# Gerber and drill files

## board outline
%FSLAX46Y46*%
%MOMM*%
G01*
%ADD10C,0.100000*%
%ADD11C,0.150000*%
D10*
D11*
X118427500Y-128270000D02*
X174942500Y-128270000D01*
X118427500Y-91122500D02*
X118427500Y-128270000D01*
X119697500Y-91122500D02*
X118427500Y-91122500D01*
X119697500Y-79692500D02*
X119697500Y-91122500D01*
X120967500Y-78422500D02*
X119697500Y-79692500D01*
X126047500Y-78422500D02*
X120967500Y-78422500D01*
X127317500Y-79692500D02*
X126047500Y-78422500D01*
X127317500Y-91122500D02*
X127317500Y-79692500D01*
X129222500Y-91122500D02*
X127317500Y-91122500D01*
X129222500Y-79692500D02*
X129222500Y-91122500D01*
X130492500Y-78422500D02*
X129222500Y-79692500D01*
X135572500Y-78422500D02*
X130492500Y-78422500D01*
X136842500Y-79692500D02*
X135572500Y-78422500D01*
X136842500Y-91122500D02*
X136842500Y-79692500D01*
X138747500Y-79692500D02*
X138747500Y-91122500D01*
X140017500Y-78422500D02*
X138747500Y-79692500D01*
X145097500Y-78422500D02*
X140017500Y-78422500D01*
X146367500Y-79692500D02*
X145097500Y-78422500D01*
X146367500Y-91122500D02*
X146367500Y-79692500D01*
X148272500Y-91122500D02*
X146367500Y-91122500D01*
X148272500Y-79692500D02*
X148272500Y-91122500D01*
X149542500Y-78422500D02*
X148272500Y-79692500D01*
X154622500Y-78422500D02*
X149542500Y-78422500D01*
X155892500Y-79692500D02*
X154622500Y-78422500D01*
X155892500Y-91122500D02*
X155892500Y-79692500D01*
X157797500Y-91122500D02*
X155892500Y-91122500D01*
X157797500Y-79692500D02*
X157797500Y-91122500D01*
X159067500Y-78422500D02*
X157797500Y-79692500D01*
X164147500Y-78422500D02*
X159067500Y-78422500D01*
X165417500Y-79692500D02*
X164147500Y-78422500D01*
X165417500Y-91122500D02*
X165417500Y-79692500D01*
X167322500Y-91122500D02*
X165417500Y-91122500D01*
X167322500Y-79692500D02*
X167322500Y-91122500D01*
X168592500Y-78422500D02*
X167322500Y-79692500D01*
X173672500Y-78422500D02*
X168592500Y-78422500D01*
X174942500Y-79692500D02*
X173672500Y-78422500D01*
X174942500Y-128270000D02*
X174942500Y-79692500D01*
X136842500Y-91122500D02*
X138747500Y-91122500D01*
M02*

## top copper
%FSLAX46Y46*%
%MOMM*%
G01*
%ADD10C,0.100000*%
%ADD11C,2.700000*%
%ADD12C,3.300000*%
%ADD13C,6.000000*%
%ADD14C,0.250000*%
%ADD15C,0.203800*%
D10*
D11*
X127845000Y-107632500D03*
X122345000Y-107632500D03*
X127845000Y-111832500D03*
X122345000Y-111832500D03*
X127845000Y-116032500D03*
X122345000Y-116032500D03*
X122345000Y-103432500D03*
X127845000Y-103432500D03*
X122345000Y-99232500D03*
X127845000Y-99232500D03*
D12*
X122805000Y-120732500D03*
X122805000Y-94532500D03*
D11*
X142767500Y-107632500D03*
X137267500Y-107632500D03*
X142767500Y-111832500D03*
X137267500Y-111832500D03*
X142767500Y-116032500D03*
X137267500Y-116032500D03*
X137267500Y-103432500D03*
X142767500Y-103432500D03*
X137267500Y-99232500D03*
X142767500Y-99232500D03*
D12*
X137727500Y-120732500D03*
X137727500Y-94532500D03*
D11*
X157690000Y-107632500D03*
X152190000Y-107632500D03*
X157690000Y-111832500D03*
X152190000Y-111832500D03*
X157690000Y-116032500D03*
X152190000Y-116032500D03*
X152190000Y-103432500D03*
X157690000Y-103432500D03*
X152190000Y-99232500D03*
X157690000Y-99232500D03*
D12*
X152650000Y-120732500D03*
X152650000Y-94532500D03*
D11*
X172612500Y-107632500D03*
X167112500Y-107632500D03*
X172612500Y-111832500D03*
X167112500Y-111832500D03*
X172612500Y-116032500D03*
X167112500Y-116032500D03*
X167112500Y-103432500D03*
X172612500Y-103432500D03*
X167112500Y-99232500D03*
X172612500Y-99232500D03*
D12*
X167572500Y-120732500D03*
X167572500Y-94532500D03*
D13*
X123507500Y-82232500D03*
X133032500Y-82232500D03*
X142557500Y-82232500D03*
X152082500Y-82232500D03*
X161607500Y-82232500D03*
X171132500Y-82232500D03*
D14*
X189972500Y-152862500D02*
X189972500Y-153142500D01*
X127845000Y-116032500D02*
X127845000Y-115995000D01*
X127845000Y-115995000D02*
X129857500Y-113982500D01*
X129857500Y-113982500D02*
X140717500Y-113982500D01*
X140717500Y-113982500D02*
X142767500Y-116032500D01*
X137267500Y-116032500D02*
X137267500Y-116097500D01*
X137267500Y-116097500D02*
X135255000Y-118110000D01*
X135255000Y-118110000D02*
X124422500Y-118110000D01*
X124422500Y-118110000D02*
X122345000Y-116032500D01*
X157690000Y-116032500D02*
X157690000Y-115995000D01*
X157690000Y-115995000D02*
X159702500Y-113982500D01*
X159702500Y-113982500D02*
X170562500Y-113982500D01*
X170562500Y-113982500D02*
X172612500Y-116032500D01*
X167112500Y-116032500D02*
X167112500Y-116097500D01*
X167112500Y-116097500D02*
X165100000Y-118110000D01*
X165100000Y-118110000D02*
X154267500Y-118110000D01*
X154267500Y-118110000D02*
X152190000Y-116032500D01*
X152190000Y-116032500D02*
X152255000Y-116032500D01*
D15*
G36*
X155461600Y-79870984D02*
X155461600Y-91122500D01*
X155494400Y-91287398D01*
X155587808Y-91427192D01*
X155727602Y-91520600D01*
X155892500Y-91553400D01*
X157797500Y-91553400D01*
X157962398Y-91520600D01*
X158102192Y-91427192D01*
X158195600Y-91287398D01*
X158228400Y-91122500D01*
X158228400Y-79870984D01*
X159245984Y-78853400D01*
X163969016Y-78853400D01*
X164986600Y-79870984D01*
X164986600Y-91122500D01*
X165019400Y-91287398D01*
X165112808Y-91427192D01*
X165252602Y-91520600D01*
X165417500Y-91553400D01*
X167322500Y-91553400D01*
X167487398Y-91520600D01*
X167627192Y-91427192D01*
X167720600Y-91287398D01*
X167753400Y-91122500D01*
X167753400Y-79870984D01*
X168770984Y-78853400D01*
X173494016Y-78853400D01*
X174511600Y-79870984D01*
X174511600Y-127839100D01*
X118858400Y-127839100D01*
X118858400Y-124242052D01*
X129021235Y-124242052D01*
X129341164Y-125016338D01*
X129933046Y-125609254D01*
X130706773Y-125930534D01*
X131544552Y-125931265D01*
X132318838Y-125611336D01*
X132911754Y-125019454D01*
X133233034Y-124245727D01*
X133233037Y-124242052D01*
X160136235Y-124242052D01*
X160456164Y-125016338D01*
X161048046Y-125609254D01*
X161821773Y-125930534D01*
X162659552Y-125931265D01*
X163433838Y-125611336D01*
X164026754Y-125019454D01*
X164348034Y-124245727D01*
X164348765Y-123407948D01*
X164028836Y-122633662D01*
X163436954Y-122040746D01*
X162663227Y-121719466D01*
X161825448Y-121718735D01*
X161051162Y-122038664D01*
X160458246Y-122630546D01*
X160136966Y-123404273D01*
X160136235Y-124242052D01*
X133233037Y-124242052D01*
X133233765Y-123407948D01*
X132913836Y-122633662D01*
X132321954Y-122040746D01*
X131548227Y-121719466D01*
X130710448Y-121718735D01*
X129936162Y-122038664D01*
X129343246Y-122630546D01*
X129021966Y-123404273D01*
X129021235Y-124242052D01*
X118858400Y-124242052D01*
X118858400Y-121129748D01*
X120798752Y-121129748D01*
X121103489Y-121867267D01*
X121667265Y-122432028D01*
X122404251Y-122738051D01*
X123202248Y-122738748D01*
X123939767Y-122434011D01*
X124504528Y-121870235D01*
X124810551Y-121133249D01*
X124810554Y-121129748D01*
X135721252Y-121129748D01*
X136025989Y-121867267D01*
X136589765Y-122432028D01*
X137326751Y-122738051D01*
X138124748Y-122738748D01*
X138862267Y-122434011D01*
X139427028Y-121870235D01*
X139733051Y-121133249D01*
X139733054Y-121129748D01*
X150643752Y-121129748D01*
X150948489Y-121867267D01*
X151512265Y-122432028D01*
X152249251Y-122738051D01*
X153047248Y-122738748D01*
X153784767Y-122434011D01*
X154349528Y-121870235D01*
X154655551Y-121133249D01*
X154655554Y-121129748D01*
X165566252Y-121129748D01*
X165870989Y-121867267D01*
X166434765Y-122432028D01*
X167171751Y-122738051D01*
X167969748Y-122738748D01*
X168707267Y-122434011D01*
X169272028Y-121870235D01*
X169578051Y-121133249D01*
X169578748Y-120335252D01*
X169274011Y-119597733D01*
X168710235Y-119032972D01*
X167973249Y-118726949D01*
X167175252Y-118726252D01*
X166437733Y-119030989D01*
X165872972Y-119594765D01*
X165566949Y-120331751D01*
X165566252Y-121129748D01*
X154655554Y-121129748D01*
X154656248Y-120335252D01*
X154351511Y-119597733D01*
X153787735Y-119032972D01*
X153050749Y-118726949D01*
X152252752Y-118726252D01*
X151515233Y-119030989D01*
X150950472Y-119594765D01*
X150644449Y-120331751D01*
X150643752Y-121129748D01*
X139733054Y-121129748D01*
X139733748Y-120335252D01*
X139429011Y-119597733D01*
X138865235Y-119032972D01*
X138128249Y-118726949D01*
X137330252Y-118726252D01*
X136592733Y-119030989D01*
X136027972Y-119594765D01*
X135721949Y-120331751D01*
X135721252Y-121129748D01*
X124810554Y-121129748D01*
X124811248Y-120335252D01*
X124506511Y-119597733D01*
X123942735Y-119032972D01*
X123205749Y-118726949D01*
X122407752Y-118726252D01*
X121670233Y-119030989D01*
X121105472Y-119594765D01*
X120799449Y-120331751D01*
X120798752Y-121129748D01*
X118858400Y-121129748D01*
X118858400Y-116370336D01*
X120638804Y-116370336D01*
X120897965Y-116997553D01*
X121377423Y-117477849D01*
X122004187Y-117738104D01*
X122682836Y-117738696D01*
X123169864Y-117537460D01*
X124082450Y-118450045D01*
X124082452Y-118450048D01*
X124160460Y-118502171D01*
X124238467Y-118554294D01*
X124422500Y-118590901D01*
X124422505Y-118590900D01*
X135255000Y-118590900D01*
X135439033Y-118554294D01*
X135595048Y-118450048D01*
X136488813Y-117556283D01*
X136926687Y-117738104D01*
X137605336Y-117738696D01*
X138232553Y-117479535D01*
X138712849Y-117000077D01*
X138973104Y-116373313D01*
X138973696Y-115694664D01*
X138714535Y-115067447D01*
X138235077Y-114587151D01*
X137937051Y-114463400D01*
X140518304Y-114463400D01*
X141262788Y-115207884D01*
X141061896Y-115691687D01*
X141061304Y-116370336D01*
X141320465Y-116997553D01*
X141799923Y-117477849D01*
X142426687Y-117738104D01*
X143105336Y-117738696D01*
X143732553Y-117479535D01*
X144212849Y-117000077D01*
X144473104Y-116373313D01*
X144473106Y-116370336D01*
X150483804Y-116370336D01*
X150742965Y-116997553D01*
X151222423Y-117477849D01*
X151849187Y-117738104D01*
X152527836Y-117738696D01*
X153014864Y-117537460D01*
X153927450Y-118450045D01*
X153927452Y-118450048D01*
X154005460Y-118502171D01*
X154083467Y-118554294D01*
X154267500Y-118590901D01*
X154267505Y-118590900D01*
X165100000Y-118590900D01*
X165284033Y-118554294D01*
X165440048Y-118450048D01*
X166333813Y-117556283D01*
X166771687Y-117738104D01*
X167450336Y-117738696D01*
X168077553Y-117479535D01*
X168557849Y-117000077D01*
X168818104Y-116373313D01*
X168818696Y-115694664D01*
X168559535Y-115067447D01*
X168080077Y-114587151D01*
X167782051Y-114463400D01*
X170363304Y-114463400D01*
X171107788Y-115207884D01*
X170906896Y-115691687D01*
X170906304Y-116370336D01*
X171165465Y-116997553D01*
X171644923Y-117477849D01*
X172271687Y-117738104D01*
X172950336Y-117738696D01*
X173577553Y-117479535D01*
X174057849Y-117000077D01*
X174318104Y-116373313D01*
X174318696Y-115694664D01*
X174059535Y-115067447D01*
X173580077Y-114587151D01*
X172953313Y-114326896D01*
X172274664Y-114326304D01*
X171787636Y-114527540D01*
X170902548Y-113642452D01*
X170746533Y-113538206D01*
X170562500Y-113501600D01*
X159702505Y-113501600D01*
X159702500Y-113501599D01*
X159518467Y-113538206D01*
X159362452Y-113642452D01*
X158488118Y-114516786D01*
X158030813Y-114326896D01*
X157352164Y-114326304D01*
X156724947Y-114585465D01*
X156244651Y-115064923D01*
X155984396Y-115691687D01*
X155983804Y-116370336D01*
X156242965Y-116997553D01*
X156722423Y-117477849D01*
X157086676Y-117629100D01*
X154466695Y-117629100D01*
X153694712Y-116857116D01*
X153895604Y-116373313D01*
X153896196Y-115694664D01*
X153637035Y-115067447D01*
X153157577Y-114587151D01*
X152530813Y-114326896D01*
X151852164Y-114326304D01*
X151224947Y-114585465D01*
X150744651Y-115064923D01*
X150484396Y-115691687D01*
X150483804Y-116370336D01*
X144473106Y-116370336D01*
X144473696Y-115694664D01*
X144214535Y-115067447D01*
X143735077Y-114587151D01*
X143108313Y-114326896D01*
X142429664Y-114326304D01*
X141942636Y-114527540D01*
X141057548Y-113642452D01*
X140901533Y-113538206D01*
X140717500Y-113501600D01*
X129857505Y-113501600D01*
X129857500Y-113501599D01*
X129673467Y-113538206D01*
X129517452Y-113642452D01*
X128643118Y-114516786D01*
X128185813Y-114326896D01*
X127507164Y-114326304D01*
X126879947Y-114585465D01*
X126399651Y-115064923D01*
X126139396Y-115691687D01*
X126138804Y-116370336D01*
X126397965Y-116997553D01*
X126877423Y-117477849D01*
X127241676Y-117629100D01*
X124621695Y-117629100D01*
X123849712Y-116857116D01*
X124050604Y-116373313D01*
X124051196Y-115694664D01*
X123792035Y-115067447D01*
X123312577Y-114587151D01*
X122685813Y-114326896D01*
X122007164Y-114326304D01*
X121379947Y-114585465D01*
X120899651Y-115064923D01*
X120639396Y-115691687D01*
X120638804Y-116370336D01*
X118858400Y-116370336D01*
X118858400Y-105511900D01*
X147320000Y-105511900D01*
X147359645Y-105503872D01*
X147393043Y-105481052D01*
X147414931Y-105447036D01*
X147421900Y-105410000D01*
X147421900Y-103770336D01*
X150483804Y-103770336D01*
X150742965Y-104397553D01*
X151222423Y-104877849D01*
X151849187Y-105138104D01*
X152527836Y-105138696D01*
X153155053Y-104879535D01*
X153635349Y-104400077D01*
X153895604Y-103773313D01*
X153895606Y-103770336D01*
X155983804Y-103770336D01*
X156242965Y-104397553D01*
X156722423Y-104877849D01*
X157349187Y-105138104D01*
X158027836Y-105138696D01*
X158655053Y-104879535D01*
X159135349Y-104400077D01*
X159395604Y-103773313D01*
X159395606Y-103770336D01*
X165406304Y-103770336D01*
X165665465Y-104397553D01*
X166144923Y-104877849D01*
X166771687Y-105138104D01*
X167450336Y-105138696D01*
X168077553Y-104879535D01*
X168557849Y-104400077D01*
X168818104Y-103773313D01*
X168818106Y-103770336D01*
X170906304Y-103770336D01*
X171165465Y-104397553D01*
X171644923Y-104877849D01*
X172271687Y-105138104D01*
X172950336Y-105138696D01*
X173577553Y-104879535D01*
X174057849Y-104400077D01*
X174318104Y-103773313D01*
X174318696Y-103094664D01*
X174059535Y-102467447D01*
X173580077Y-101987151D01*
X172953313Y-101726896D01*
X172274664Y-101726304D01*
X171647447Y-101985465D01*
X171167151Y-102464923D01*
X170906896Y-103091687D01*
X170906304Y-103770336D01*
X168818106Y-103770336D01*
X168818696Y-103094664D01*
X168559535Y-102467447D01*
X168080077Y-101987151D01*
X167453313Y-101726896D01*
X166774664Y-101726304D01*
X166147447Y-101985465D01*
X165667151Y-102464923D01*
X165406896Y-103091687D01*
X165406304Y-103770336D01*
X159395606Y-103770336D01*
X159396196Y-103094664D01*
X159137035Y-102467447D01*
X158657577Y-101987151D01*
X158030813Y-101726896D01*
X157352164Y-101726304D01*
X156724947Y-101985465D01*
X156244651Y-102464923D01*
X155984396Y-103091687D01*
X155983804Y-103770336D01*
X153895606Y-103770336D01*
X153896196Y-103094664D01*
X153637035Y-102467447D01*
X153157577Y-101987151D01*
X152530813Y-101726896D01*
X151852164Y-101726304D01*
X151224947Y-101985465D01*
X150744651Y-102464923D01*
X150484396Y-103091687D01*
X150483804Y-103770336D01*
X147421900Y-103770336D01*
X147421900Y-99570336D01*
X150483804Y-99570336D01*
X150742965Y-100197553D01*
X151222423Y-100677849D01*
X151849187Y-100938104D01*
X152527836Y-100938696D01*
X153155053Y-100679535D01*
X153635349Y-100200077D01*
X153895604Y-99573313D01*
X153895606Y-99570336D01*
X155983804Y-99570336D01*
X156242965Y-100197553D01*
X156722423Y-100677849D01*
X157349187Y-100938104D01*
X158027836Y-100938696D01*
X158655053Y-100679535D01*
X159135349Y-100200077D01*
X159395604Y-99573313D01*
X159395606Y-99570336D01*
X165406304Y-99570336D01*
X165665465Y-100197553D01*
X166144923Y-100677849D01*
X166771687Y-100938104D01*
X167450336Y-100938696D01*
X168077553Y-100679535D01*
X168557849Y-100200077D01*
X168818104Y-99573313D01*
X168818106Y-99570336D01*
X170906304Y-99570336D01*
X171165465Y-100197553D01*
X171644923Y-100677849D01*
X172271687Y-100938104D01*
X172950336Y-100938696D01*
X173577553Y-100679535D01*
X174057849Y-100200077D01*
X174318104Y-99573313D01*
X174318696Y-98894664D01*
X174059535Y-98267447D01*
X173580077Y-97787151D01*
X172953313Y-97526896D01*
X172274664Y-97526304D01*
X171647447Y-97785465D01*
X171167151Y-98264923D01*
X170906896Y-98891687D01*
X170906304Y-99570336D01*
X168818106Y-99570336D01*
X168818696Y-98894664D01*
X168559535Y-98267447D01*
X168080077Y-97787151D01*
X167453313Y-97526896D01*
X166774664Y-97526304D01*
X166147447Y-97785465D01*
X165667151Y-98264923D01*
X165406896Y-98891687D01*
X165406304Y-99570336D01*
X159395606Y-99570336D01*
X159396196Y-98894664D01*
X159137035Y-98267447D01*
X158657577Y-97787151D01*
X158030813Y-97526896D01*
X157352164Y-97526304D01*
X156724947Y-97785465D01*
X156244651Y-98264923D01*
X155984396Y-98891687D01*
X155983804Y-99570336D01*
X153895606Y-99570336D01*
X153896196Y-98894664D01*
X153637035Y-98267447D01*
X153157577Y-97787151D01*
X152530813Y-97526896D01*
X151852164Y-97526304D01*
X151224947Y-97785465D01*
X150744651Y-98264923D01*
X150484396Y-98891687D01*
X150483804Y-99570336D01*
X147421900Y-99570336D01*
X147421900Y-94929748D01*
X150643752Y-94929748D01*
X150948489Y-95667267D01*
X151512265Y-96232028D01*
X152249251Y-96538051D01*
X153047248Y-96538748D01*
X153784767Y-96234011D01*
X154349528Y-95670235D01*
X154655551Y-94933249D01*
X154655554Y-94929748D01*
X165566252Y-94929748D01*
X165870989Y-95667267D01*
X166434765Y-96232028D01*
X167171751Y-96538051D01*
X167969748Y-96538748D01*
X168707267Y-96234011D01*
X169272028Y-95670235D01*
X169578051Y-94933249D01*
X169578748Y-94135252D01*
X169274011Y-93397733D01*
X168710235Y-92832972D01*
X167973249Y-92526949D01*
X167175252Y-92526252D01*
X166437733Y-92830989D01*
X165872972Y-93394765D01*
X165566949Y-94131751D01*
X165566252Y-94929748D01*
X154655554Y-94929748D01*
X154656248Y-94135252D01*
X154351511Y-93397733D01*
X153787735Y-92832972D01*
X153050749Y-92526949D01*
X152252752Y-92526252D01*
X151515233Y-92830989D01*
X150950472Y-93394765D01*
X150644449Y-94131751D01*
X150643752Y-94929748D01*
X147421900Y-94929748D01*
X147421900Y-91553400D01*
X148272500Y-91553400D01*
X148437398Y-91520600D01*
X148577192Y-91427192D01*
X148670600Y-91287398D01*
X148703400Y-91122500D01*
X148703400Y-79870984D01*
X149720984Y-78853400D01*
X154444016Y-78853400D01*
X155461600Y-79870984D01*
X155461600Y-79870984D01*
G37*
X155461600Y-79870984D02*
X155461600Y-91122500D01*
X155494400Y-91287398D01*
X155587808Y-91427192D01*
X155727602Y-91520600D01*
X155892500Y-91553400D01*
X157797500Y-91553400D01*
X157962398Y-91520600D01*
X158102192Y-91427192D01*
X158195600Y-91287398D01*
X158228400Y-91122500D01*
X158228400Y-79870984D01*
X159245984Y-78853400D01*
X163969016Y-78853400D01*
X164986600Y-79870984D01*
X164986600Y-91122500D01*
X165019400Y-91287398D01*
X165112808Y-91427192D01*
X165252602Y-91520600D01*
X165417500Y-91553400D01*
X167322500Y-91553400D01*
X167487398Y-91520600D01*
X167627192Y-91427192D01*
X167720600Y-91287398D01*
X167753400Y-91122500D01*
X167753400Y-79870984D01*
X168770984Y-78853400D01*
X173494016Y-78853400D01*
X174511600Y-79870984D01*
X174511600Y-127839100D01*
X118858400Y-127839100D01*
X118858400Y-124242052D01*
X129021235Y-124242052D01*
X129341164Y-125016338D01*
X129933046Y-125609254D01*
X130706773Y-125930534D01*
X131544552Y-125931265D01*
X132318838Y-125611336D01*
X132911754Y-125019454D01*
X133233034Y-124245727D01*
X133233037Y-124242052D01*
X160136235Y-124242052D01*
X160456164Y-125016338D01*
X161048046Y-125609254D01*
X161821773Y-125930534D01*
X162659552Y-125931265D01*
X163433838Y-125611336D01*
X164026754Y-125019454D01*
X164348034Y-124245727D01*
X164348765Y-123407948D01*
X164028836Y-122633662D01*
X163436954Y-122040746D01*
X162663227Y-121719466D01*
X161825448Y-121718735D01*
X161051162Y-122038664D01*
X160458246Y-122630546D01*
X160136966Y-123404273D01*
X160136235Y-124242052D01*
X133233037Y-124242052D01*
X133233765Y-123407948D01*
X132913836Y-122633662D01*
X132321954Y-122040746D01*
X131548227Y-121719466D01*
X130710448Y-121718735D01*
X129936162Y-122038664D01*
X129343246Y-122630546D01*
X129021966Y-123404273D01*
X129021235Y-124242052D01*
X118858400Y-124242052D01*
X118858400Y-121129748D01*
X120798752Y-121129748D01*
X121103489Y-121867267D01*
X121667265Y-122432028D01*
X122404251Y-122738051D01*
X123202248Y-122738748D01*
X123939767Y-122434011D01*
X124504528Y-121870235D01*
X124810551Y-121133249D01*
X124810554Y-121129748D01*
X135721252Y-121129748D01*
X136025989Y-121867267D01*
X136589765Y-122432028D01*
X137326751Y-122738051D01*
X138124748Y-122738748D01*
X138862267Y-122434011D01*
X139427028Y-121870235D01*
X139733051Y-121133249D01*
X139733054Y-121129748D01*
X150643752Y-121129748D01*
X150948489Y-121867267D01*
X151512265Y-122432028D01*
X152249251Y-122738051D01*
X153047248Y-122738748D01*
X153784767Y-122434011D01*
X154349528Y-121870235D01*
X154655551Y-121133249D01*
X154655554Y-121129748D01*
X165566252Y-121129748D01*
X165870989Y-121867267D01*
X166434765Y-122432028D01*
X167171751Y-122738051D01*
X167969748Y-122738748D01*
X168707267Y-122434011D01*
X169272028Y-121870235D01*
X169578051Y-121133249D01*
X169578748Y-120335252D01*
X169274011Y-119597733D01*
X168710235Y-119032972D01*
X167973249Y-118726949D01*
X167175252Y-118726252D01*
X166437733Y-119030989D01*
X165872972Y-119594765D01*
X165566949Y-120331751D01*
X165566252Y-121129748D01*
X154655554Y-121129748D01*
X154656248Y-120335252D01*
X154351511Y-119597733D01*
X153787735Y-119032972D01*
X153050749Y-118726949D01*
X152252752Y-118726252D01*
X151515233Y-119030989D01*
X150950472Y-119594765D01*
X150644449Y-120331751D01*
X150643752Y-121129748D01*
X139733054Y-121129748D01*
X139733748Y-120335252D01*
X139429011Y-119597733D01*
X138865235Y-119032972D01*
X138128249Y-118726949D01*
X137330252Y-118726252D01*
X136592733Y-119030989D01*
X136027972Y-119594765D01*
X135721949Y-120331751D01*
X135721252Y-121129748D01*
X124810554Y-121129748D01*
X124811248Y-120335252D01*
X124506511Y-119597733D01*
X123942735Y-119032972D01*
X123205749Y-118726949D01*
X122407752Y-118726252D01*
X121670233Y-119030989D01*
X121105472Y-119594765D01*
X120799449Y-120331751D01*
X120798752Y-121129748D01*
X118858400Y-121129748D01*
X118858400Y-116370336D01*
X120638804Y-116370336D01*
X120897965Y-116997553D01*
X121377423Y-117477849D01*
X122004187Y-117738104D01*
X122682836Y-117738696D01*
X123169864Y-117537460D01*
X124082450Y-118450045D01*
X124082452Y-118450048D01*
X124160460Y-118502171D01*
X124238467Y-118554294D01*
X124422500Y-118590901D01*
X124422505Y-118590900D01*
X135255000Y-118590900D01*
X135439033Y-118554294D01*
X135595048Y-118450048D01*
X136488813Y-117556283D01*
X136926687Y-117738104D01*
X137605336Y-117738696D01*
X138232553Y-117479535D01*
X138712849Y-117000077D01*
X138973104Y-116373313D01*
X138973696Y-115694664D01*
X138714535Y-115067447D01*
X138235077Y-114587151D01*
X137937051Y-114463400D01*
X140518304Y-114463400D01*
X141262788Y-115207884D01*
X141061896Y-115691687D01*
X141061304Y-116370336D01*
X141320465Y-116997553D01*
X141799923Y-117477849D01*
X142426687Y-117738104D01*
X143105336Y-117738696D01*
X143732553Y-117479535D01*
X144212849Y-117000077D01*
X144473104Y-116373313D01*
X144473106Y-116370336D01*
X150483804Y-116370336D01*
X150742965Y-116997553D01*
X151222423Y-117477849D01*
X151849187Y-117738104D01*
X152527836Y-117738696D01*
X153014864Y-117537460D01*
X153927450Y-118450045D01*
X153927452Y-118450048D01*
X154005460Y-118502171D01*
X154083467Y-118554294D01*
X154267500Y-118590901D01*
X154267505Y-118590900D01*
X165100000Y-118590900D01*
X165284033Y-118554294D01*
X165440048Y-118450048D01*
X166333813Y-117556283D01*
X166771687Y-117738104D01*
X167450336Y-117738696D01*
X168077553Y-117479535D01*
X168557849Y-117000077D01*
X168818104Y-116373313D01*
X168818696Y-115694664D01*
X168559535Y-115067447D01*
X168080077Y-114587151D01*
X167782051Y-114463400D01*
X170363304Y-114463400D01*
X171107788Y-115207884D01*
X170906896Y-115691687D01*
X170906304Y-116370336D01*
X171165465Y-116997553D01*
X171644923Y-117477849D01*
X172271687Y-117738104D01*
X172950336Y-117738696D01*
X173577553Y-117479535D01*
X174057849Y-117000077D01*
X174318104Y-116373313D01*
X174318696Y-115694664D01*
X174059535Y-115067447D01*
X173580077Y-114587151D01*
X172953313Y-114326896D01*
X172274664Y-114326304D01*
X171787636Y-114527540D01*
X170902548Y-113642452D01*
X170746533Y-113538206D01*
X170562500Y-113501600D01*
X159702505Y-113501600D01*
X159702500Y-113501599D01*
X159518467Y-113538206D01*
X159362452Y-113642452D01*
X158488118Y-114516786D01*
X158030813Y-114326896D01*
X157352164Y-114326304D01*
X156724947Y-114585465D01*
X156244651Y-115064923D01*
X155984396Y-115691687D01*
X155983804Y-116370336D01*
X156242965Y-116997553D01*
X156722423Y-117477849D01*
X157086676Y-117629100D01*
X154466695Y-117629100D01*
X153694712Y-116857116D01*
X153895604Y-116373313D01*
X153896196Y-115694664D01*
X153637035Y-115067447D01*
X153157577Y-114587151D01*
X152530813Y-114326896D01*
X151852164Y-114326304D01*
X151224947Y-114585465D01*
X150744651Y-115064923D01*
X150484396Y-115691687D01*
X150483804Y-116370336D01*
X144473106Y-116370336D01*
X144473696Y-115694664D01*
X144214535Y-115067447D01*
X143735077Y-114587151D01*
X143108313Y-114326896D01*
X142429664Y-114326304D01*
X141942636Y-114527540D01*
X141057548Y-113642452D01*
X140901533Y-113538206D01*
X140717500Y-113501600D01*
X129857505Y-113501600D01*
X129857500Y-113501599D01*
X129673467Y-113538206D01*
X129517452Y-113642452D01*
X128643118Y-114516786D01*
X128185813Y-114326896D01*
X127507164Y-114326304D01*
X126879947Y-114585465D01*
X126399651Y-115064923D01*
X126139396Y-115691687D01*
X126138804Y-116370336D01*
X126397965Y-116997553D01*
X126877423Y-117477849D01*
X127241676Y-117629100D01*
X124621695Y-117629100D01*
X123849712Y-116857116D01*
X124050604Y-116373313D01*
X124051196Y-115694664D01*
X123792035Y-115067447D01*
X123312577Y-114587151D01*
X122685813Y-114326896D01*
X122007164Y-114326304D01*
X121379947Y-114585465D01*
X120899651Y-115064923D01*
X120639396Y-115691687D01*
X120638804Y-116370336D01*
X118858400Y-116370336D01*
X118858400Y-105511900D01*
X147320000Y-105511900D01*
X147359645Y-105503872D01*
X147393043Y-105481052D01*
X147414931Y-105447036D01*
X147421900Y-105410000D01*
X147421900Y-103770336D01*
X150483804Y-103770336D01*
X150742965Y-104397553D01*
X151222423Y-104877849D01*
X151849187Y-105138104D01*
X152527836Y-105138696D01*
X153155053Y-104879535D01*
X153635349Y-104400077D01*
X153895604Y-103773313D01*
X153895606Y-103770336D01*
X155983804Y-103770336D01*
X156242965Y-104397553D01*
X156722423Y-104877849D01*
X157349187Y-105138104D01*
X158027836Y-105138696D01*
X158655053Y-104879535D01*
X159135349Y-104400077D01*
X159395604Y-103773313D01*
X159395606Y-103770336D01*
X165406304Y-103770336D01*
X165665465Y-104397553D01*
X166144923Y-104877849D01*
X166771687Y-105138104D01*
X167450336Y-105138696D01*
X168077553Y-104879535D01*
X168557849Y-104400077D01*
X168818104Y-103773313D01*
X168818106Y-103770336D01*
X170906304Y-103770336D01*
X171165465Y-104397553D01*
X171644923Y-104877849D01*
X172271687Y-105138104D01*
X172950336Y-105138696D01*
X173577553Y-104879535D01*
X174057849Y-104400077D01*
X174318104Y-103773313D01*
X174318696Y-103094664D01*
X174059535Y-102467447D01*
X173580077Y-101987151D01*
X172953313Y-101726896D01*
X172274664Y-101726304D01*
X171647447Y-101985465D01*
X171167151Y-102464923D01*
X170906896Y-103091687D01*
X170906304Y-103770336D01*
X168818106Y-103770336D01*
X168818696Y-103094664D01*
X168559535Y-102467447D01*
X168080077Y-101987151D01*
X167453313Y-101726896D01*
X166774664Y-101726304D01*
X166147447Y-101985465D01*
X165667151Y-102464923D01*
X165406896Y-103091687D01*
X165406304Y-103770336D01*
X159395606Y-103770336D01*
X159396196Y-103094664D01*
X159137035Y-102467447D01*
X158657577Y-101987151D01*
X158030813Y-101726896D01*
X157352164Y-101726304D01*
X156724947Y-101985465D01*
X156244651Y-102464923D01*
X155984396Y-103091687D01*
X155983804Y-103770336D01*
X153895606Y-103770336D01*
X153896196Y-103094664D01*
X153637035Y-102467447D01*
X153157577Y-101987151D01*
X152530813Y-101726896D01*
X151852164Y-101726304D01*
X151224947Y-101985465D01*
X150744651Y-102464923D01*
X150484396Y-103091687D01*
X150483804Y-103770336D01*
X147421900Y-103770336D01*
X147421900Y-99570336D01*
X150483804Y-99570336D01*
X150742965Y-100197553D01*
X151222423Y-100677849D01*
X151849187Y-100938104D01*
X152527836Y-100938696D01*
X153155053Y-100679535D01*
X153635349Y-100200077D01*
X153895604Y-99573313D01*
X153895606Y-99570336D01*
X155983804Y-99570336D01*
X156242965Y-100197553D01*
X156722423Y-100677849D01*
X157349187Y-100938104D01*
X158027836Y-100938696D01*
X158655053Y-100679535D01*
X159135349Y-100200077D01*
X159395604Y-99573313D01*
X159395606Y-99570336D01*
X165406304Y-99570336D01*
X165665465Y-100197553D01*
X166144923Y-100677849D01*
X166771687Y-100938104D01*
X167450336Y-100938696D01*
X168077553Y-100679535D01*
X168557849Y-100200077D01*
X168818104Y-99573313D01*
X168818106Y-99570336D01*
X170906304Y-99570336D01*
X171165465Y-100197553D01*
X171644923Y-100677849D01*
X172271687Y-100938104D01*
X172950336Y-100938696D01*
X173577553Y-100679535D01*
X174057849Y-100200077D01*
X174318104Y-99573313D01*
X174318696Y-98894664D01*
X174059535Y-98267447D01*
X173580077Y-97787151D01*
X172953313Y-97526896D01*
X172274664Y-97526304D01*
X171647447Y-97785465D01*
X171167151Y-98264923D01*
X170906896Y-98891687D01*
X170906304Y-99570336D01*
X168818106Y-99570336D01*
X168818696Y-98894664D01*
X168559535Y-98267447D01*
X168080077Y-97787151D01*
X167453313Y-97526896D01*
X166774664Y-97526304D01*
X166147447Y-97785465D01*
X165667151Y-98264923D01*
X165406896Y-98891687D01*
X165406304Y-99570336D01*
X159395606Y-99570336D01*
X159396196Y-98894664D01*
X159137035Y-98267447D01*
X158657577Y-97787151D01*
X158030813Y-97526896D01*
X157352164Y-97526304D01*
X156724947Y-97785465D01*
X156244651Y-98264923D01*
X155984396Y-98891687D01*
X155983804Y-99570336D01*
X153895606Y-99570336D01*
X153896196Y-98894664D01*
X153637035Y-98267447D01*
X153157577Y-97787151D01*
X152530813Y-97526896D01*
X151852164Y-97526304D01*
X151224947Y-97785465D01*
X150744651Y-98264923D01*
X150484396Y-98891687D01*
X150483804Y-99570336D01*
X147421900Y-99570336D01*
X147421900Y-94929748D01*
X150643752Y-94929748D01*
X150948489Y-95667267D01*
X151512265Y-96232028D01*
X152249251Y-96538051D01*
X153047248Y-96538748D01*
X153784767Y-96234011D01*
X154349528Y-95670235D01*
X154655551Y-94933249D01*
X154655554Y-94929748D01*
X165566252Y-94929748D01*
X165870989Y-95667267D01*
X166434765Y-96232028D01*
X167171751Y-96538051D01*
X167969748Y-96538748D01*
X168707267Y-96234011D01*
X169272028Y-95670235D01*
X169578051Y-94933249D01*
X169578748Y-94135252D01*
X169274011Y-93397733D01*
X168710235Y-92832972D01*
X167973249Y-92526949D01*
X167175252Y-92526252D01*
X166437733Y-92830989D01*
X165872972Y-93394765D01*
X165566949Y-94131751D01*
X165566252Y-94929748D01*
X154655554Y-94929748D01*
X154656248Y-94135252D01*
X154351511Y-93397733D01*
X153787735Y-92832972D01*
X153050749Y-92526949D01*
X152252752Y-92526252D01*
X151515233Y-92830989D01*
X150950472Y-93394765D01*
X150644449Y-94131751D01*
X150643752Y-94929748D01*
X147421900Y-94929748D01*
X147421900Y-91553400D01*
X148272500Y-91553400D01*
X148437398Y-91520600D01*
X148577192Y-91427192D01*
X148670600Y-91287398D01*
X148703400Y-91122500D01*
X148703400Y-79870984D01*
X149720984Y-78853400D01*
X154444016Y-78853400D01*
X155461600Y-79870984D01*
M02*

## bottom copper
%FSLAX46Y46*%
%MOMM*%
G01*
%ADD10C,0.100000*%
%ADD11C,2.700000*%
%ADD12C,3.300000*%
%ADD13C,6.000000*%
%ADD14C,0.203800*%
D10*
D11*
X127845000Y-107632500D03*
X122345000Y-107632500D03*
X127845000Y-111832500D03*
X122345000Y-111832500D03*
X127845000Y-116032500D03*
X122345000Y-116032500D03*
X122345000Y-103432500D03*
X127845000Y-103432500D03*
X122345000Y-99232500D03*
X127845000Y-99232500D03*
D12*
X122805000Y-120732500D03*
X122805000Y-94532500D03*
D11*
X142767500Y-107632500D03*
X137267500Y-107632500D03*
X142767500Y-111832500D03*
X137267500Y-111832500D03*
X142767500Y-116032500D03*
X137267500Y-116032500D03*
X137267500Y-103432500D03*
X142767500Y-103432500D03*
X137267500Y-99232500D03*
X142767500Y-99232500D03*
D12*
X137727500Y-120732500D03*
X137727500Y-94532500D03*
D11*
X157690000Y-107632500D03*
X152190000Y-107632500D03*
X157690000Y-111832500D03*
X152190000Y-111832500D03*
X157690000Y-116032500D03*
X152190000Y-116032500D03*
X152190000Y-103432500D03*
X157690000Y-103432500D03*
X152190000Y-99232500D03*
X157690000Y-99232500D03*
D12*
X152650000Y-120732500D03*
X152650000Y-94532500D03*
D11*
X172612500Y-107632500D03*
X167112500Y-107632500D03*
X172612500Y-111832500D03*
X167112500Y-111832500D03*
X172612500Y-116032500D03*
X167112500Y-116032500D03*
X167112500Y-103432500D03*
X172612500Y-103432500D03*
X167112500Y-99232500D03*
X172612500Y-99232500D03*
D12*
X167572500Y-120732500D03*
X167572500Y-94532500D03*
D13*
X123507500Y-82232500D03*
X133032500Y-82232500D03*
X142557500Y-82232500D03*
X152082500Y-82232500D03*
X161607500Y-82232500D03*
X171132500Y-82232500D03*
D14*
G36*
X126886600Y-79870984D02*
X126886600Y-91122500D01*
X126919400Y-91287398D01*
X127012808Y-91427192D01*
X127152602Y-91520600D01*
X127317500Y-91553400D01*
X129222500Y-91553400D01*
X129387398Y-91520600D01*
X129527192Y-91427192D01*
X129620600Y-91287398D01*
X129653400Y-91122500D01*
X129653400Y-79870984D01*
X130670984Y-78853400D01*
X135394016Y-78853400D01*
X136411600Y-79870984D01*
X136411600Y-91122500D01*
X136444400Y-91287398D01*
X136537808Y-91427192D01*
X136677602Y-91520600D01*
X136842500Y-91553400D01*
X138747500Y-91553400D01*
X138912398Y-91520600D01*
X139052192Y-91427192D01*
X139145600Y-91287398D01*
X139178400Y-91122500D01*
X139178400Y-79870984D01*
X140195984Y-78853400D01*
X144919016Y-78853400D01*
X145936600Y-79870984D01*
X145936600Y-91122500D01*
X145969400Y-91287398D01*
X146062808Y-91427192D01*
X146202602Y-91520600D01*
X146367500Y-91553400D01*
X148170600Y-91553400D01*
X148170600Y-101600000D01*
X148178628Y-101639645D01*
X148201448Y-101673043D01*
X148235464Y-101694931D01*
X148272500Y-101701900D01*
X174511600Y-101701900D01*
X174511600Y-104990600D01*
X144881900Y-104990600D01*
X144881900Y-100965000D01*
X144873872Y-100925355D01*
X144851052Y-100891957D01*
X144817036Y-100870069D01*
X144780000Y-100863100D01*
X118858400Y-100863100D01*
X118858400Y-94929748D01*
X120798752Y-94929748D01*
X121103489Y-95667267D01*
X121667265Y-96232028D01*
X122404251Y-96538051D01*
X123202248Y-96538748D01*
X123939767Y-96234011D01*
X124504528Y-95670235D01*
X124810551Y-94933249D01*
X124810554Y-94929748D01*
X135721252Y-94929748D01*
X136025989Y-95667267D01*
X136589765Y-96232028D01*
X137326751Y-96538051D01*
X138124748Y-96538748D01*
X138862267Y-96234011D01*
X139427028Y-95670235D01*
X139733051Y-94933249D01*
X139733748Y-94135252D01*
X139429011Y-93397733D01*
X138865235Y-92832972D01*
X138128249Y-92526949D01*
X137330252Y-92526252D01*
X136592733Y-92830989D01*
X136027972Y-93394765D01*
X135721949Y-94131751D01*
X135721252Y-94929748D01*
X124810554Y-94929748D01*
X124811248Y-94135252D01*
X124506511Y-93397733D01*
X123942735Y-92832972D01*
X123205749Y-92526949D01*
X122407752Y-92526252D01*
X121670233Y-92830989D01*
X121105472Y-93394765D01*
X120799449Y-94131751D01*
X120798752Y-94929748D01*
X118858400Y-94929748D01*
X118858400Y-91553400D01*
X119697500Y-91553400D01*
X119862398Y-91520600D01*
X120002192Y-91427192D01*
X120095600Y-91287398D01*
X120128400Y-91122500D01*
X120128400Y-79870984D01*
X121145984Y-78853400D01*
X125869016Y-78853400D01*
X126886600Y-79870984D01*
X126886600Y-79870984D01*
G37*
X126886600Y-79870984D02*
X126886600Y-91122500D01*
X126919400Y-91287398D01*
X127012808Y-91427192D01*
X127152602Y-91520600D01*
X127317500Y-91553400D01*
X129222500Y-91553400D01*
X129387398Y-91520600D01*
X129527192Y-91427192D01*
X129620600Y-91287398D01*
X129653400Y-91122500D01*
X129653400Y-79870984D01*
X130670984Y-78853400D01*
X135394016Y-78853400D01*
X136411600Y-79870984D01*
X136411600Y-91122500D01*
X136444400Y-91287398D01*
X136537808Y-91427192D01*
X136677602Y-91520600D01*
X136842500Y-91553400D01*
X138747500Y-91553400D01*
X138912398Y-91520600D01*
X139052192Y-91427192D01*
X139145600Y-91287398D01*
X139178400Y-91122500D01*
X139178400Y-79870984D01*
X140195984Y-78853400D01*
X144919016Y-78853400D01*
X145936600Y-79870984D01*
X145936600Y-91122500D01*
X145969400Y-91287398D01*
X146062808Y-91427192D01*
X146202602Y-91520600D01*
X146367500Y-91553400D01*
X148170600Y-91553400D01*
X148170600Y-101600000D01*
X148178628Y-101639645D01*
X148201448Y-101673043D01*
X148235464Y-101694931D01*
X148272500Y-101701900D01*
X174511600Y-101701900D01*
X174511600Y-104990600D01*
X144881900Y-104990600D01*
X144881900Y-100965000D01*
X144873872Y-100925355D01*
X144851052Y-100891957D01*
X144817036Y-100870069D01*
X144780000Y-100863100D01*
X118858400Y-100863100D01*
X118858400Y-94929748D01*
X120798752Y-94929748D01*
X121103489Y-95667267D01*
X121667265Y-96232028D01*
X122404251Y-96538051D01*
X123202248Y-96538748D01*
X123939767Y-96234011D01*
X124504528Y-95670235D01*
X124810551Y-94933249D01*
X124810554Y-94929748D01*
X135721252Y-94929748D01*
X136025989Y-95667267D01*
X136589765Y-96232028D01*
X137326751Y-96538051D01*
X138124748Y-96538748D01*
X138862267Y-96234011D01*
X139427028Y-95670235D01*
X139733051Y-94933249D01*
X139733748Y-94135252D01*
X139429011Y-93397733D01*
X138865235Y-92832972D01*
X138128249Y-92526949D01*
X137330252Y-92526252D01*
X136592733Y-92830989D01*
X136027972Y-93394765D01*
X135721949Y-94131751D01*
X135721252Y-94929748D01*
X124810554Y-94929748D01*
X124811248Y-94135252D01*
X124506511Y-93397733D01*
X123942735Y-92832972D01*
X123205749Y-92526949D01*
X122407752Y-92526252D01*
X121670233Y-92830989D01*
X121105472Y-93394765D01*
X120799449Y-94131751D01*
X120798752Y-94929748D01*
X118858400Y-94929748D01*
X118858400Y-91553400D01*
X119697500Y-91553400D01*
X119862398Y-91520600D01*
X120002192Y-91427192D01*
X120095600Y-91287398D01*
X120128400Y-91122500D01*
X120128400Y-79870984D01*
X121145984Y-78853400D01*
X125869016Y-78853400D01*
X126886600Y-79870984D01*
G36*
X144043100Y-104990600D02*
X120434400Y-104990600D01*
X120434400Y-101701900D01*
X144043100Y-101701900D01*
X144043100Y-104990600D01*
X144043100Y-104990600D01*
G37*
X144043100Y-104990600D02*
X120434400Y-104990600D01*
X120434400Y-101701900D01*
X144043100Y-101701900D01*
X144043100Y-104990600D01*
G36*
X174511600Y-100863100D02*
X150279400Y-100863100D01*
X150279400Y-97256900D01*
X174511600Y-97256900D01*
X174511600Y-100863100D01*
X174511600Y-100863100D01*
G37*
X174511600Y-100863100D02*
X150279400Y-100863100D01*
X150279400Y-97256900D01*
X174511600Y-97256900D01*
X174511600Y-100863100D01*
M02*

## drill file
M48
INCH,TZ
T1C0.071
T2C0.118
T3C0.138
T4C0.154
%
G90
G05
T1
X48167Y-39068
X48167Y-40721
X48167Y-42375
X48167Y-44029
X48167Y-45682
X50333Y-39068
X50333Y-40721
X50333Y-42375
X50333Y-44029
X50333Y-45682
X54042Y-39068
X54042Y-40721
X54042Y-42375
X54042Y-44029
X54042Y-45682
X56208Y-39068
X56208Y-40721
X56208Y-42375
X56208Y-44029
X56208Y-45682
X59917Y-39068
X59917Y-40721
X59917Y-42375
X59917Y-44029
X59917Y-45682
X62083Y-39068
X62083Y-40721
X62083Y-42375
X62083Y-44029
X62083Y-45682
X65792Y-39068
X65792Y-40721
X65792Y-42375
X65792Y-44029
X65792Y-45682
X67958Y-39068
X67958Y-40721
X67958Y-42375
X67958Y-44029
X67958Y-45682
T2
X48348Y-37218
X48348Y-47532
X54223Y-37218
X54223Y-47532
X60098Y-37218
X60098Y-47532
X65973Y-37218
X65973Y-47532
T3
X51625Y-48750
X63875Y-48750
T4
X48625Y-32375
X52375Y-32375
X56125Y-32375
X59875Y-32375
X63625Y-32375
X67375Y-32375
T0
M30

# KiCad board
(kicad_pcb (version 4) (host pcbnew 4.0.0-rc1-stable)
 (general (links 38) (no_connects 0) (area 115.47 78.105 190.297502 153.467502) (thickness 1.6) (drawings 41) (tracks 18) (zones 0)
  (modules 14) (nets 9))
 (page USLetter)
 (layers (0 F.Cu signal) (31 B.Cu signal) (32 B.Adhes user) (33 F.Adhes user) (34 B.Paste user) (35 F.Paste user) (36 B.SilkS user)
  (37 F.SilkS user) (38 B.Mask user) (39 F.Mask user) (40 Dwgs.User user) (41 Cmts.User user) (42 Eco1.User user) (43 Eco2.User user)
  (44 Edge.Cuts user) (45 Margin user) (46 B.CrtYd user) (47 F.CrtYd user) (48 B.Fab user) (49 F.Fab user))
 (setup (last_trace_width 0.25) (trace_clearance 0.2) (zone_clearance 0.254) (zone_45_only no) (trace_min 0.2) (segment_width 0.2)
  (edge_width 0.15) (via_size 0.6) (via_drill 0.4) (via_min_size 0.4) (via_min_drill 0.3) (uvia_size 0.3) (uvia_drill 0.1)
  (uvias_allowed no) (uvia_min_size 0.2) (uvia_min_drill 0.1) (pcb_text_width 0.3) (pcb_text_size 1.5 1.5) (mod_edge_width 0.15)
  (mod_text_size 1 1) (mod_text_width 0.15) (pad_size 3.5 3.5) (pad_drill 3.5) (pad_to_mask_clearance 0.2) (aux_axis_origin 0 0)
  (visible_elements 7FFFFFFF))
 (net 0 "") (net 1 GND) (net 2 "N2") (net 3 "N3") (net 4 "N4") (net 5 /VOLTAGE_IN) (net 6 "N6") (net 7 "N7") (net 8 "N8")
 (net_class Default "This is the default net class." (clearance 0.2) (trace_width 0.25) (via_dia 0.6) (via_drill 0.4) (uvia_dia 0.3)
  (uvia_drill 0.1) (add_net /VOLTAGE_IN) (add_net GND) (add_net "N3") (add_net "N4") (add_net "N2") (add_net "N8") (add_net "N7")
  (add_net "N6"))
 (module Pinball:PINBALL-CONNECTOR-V (layer F.Cu) (at 125.095 107.6325 270)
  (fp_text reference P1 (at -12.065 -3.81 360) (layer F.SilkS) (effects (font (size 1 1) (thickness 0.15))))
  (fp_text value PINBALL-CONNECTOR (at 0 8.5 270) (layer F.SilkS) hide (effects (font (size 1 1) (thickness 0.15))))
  (pad 3 thru_hole circle (at 0 -2.75 90) (size 2.7 2.7) (drill 1.8) (layers *.Cu *.Mask F.SilkS) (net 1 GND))
  (pad 8 thru_hole circle (at 0 2.75 90) (size 2.7 2.7) (drill 1.8) (layers *.Cu *.Mask F.SilkS) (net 1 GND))
  (pad 4 thru_hole circle (at 4.2 -2.75 90) (size 2.7 2.7) (drill 1.8) (layers *.Cu *.Mask F.SilkS) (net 1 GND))
  (pad 9 thru_hole circle (at 4.2 2.75 90) (size 2.7 2.7) (drill 1.8) (layers *.Cu *.Mask F.SilkS) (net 1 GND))
  (pad 5 thru_hole circle (at 8.4 -2.75 90) (size 2.7 2.7) (drill 1.8) (layers *.Cu *.Mask F.SilkS) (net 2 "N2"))
  (pad 10 thru_hole circle (at 8.4 2.75 90) (size 2.7 2.7) (drill 1.8) (layers *.Cu *.Mask F.SilkS) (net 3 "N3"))
  (pad 7 thru_hole circle (at -4.2 2.75 90) (size 2.7 2.7) (drill 1.8) (layers *.Cu *.Mask F.SilkS) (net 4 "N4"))
  (pad 2 thru_hole circle (at -4.2 -2.75 90) (size 2.7 2.7) (drill 1.8) (layers *.Cu *.Mask F.SilkS) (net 4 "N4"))
  (pad 6 thru_hole circle (at -8.4 2.75 90) (size 2.7 2.7) (drill 1.8) (layers *.Cu *.Mask F.SilkS) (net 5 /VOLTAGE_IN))
  (pad 1 thru_hole circle (at -8.4 -2.75 90) (size 2.7 2.7) (drill 1.8) (layers *.Cu *.Mask F.SilkS) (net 5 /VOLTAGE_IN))
  (pad "" np_thru_hole circle (at 13.1 2.29 90) (size 3.3 3.3) (drill 3) (layers *.Cu *.Mask F.SilkS))
  (pad "" np_thru_hole circle (at -13.1 2.29 90) (size 3.3 3.3) (drill 3) (layers *.Cu *.Mask F.SilkS)))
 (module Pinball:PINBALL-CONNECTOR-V (layer F.Cu) (at 140.0175 107.6325 270)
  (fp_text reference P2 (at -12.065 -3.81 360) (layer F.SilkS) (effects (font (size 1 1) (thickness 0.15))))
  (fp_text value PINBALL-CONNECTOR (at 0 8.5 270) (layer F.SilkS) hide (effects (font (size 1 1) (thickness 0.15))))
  (pad 3 thru_hole circle (at 0 -2.75 90) (size 2.7 2.7) (drill 1.8) (layers *.Cu *.Mask F.SilkS) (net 1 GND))
  (pad 8 thru_hole circle (at 0 2.75 90) (size 2.7 2.7) (drill 1.8) (layers *.Cu *.Mask F.SilkS) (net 1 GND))
  (pad 4 thru_hole circle (at 4.2 -2.75 90) (size 2.7 2.7) (drill 1.8) (layers *.Cu *.Mask F.SilkS) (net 1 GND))
  (pad 9 thru_hole circle (at 4.2 2.75 90) (size 2.7 2.7) (drill 1.8) (layers *.Cu *.Mask F.SilkS) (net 1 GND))
  (pad 5 thru_hole circle (at 8.4 -2.75 90) (size 2.7 2.7) (drill 1.8) (layers *.Cu *.Mask F.SilkS) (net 2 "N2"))
  (pad 10 thru_hole circle (at 8.4 2.75 90) (size 2.7 2.7) (drill 1.8) (layers *.Cu *.Mask F.SilkS) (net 3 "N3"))
  (pad 7 thru_hole circle (at -4.2 2.75 90) (size 2.7 2.7) (drill 1.8) (layers *.Cu *.Mask F.SilkS) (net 4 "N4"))
  (pad 2 thru_hole circle (at -4.2 -2.75 90) (size 2.7 2.7) (drill 1.8) (layers *.Cu *.Mask F.SilkS) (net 4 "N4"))
  (pad 6 thru_hole circle (at -8.4 2.75 90) (size 2.7 2.7) (drill 1.8) (layers *.Cu *.Mask F.SilkS) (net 5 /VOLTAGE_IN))
  (pad 1 thru_hole circle (at -8.4 -2.75 90) (size 2.7 2.7) (drill 1.8) (layers *.Cu *.Mask F.SilkS) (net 5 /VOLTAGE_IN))
  (pad "" np_thru_hole circle (at 13.1 2.29 90) (size 3.3 3.3) (drill 3) (layers *.Cu *.Mask F.SilkS))
  (pad "" np_thru_hole circle (at -13.1 2.29 90) (size 3.3 3.3) (drill 3) (layers *.Cu *.Mask F.SilkS)))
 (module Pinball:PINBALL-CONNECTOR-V (layer F.Cu) (at 154.94 107.6325 270)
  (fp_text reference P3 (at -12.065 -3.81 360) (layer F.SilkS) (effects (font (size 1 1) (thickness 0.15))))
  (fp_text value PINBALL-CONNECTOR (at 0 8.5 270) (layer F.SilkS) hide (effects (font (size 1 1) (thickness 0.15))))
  (pad 3 thru_hole circle (at 0 -2.75 90) (size 2.7 2.7) (drill 1.8) (layers *.Cu *.Mask F.SilkS) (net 1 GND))
  (pad 8 thru_hole circle (at 0 2.75 90) (size 2.7 2.7) (drill 1.8) (layers *.Cu *.Mask F.SilkS) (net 1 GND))
  (pad 4 thru_hole circle (at 4.2 -2.75 90) (size 2.7 2.7) (drill 1.8) (layers *.Cu *.Mask F.SilkS) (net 1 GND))
  (pad 9 thru_hole circle (at 4.2 2.75 90) (size 2.7 2.7) (drill 1.8) (layers *.Cu *.Mask F.SilkS) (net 1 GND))
  (pad 5 thru_hole circle (at 8.4 -2.75 90) (size 2.7 2.7) (drill 1.8) (layers *.Cu *.Mask F.SilkS) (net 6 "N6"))
  (pad 10 thru_hole circle (at 8.4 2.75 90) (size 2.7 2.7) (drill 1.8) (layers *.Cu *.Mask F.SilkS) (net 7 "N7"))
  (pad 7 thru_hole circle (at -4.2 2.75 90) (size 2.7 2.7) (drill 1.8) (layers *.Cu *.Mask F.SilkS) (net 5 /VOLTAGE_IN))
  (pad 2 thru_hole circle (at -4.2 -2.75 90) (size 2.7 2.7) (drill 1.8) (layers *.Cu *.Mask F.SilkS) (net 5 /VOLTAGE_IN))
  (pad 6 thru_hole circle (at -8.4 2.75 90) (size 2.7 2.7) (drill 1.8) (layers *.Cu *.Mask F.SilkS) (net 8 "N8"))
  (pad 1 thru_hole circle (at -8.4 -2.75 90) (size 2.7 2.7) (drill 1.8) (layers *.Cu *.Mask F.SilkS) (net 8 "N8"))
  (pad "" np_thru_hole circle (at 13.1 2.29 90) (size 3.3 3.3) (drill 3) (layers *.Cu *.Mask F.SilkS))
  (pad "" np_thru_hole circle (at -13.1 2.29 90) (size 3.3 3.3) (drill 3) (layers *.Cu *.Mask F.SilkS)))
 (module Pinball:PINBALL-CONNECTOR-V (layer F.Cu) (at 169.8625 107.6325 270)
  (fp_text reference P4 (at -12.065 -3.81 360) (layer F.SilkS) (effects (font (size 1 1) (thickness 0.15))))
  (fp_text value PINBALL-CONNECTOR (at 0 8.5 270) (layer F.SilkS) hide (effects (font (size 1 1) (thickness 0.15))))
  (pad 3 thru_hole circle (at 0 -2.75 90) (size 2.7 2.7) (drill 1.8) (layers *.Cu *.Mask F.SilkS) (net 1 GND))
  (pad 8 thru_hole circle (at 0 2.75 90) (size 2.7 2.7) (drill 1.8) (layers *.Cu *.Mask F.SilkS) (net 1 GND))
  (pad 4 thru_hole circle (at 4.2 -2.75 90) (size 2.7 2.7) (drill 1.8) (layers *.Cu *.Mask F.SilkS) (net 1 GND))
  (pad 9 thru_hole circle (at 4.2 2.75 90) (size 2.7 2.7) (drill 1.8) (layers *.Cu *.Mask F.SilkS) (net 1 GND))
  (pad 5 thru_hole circle (at 8.4 -2.75 90) (size 2.7 2.7) (drill 1.8) (layers *.Cu *.Mask F.SilkS) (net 6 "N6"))
  (pad 10 thru_hole circle (at 8.4 2.75 90) (size 2.7 2.7) (drill 1.8) (layers *.Cu *.Mask F.SilkS) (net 7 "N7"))
  (pad 7 thru_hole circle (at -4.2 2.75 90) (size 2.7 2.7) (drill 1.8) (layers *.Cu *.Mask F.SilkS) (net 5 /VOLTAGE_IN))
  (pad 2 thru_hole circle (at -4.2 -2.75 90) (size 2.7 2.7) (drill 1.8) (layers *.Cu *.Mask F.SilkS) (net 5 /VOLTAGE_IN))
  (pad 6 thru_hole circle (at -8.4 2.75 90) (size 2.7 2.7) (drill 1.8) (layers *.Cu *.Mask F.SilkS) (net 8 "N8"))
  (pad 1 thru_hole circle (at -8.4 -2.75 90) (size 2.7 2.7) (drill 1.8) (layers *.Cu *.Mask F.SilkS) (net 8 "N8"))
  (pad "" np_thru_hole circle (at 13.1 2.29 90) (size 3.3 3.3) (drill 3) (layers *.Cu *.Mask F.SilkS))
  (pad "" np_thru_hole circle (at -13.1 2.29 90) (size 3.3 3.3) (drill 3) (layers *.Cu *.Mask F.SilkS)))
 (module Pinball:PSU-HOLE (layer F.Cu) (at 123.5075 82.2325)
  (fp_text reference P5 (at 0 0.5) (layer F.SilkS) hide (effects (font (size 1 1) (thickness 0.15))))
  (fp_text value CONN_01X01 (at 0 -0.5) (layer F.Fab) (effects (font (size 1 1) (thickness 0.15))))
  (pad 1 thru_hole circle (at 0 0) (size 6 6) (drill 3.9) (layers *.Cu *.Mask F.SilkS) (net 5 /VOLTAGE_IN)))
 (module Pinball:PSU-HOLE (layer F.Cu) (at 133.0325 82.2325)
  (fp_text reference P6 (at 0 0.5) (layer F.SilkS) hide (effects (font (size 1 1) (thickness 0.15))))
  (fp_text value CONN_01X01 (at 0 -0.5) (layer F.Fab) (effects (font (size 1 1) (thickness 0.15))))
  (pad 1 thru_hole circle (at 0 0) (size 6 6) (drill 3.9) (layers *.Cu *.Mask F.SilkS) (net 5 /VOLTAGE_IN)))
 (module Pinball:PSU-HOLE (layer F.Cu) (at 142.5575 82.2325)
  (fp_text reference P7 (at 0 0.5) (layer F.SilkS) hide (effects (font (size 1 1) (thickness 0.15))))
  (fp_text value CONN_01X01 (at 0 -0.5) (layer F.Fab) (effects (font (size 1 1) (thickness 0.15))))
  (pad 1 thru_hole circle (at 0 0) (size 6 6) (drill 3.9) (layers *.Cu *.Mask F.SilkS) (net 5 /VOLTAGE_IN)))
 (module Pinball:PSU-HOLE (layer F.Cu) (at 152.0825 82.2325)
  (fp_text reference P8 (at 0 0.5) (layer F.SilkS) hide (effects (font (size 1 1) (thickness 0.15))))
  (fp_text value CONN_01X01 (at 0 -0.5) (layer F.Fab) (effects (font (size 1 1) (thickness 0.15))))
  (pad 1 thru_hole circle (at 0 0) (size 6 6) (drill 3.9) (layers *.Cu *.Mask F.SilkS) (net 1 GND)))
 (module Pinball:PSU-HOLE (layer F.Cu) (at 161.6075 82.2325)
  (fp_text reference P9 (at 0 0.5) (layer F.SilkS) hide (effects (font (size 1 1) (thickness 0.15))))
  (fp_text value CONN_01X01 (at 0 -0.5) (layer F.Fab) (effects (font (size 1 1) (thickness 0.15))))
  (pad 1 thru_hole circle (at 0 0) (size 6 6) (drill 3.9) (layers *.Cu *.Mask F.SilkS) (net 1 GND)))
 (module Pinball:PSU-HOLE (layer F.Cu) (at 171.1325 82.2325)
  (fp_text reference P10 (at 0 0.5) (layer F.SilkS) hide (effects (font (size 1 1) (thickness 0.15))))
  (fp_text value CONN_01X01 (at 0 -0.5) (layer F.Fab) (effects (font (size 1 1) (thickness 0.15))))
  (pad 1 thru_hole circle (at 0 0) (size 6 6) (drill 3.9) (layers *.Cu *.Mask F.SilkS) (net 1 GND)))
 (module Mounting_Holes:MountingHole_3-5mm (layer F.Cu) (at 162.2425 123.825)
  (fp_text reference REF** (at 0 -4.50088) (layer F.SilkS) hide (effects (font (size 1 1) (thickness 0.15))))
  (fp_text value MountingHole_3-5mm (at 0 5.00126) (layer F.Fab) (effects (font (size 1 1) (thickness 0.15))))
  (pad 1 thru_hole circle (at 0 0) (size 3.5 3.5) (drill 3.5) (layers)))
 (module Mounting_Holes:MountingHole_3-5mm (layer F.Cu) (at 131.1275 123.825)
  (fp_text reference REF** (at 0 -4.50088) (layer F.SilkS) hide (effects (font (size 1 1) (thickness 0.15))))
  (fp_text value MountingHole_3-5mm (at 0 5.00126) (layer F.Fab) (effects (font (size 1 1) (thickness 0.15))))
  (pad 1 thru_hole circle (at 0 0) (size 3.5 3.5) (drill 3.5) (layers)))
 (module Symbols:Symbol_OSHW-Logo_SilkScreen (layer F.Cu) (at 171.1325 88.5825)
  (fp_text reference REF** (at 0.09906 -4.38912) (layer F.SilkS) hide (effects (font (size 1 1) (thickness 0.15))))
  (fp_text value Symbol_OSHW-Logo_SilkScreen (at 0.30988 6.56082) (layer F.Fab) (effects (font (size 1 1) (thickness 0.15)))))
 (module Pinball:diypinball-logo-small (layer B.Cu) (at 145.7325 123.5075 180)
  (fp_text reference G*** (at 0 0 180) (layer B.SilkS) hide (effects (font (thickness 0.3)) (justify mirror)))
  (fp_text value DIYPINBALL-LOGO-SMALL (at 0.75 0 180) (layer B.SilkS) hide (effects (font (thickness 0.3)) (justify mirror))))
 (gr_line (start 118.4275 128.27) (end 174.9425 128.27) (angle 90) (layer Edge.Cuts) (width 0.15))
 (gr_line (start 118.4275 91.1225) (end 118.4275 128.27) (angle 90) (layer Edge.Cuts) (width 0.15))
 (gr_line (start 119.6975 91.1225) (end 118.4275 91.1225) (angle 90) (layer Edge.Cuts) (width 0.15))
 (gr_line (start 119.6975 79.6925) (end 119.6975 91.1225) (angle 90) (layer Edge.Cuts) (width 0.15))
 (gr_line (start 120.9675 78.4225) (end 119.6975 79.6925) (angle 90) (layer Edge.Cuts) (width 0.15))
 (gr_line (start 126.0475 78.4225) (end 120.9675 78.4225) (angle 90) (layer Edge.Cuts) (width 0.15))
 (gr_line (start 127.3175 79.6925) (end 126.0475 78.4225) (angle 90) (layer Edge.Cuts) (width 0.15))
 (gr_line (start 127.3175 91.1225) (end 127.3175 79.6925) (angle 90) (layer Edge.Cuts) (width 0.15))
 (gr_line (start 129.2225 91.1225) (end 127.3175 91.1225) (angle 90) (layer Edge.Cuts) (width 0.15))
 (gr_line (start 129.2225 79.6925) (end 129.2225 91.1225) (angle 90) (layer Edge.Cuts) (width 0.15))
 (gr_line (start 130.4925 78.4225) (end 129.2225 79.6925) (angle 90) (layer Edge.Cuts) (width 0.15))
 (gr_line (start 135.5725 78.4225) (end 130.4925 78.4225) (angle 90) (layer Edge.Cuts) (width 0.15))
 (gr_line (start 136.8425 79.6925) (end 135.5725 78.4225) (angle 90) (layer Edge.Cuts) (width 0.15))
 (gr_line (start 136.8425 91.1225) (end 136.8425 79.6925) (angle 90) (layer Edge.Cuts) (width 0.15))
 (gr_line (start 138.7475 79.6925) (end 138.7475 91.1225) (angle 90) (layer Edge.Cuts) (width 0.15))
 (gr_line (start 140.0175 78.4225) (end 138.7475 79.6925) (angle 90) (layer Edge.Cuts) (width 0.15))
 (gr_line (start 145.0975 78.4225) (end 140.0175 78.4225) (angle 90) (layer Edge.Cuts) (width 0.15))
 (gr_line (start 146.3675 79.6925) (end 145.0975 78.4225) (angle 90) (layer Edge.Cuts) (width 0.15))
 (gr_line (start 146.3675 91.1225) (end 146.3675 79.6925) (angle 90) (layer Edge.Cuts) (width 0.15))
 (gr_line (start 148.2725 91.1225) (end 146.3675 91.1225) (angle 90) (layer Edge.Cuts) (width 0.15))
 (gr_line (start 148.2725 79.6925) (end 148.2725 91.1225) (angle 90) (layer Edge.Cuts) (width 0.15))
 (gr_line (start 149.5425 78.4225) (end 148.2725 79.6925) (angle 90) (layer Edge.Cuts) (width 0.15))
 (gr_line (start 154.6225 78.4225) (end 149.5425 78.4225) (angle 90) (layer Edge.Cuts) (width 0.15))
 (gr_line (start 155.8925 79.6925) (end 154.6225 78.4225) (angle 90) (layer Edge.Cuts) (width 0.15))
 (gr_line (start 155.8925 91.1225) (end 155.8925 79.6925) (angle 90) (layer Edge.Cuts) (width 0.15))
 (gr_line (start 157.7975 91.1225) (end 155.8925 91.1225) (angle 90) (layer Edge.Cuts) (width 0.15))
 (gr_line (start 157.7975 79.6925) (end 157.7975 91.1225) (angle 90) (layer Edge.Cuts) (width 0.15))
 (gr_line (start 159.0675 78.4225) (end 157.7975 79.6925) (angle 90) (layer Edge.Cuts) (width 0.15))
 (gr_line (start 164.1475 78.4225) (end 159.0675 78.4225) (angle 90) (layer Edge.Cuts) (width 0.15))
 (gr_line (start 165.4175 79.6925) (end 164.1475 78.4225) (angle 90) (layer Edge.Cuts) (width 0.15))
 (gr_line (start 165.4175 91.1225) (end 165.4175 79.6925) (angle 90) (layer Edge.Cuts) (width 0.15))
 (gr_line (start 167.3225 91.1225) (end 165.4175 91.1225) (angle 90) (layer Edge.Cuts) (width 0.15))
 (gr_line (start 167.3225 79.6925) (end 167.3225 91.1225) (angle 90) (layer Edge.Cuts) (width 0.15))
 (gr_line (start 168.5925 78.4225) (end 167.3225 79.6925) (angle 90) (layer Edge.Cuts) (width 0.15))
 (gr_line (start 173.6725 78.4225) (end 168.5925 78.4225) (angle 90) (layer Edge.Cuts) (width 0.15))
 (gr_line (start 174.9425 79.6925) (end 173.6725 78.4225) (angle 90) (layer Edge.Cuts) (width 0.15))
 (gr_line (start 174.9425 128.27) (end 174.9425 79.6925) (angle 90) (layer Edge.Cuts) (width 0.15))
 (gr_line (start 136.8425 91.1225) (end 138.7475 91.1225) (angle 90) (layer Edge.Cuts) (width 0.15))
 (segment (start 189.9725 152.8625) (end 189.9725 153.1425) (width 0.25) (layer F.Cu) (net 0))
 (segment (start 127.845 116.0325) (end 127.845 115.995) (width 0.25) (layer F.Cu) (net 2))
 (segment (start 127.845 115.995) (end 129.8575 113.9825) (width 0.25) (layer F.Cu) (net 2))
 (segment (start 129.8575 113.9825) (end 140.7175 113.9825) (width 0.25) (layer F.Cu) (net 2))
 (segment (start 140.7175 113.9825) (end 142.7675 116.0325) (width 0.25) (layer F.Cu) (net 2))
 (segment (start 137.2675 116.0325) (end 137.2675 116.0975) (width 0.25) (layer F.Cu) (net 3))
 (segment (start 137.2675 116.0975) (end 135.255 118.11) (width 0.25) (layer F.Cu) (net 3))
 (segment (start 135.255 118.11) (end 124.4225 118.11) (width 0.25) (layer F.Cu) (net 3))
 (segment (start 124.4225 118.11) (end 122.345 116.0325) (width 0.25) (layer F.Cu) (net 3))
 (segment (start 157.69 116.0325) (end 157.69 115.995) (width 0.25) (layer F.Cu) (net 6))
 (segment (start 157.69 115.995) (end 159.7025 113.9825) (width 0.25) (layer F.Cu) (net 6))
 (segment (start 159.7025 113.9825) (end 170.5625 113.9825) (width 0.25) (layer F.Cu) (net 6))
 (segment (start 170.5625 113.9825) (end 172.6125 116.0325) (width 0.25) (layer F.Cu) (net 6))
 (segment (start 167.1125 116.0325) (end 167.1125 116.0975) (width 0.25) (layer F.Cu) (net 7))
 (segment (start 167.1125 116.0975) (end 165.1 118.11) (width 0.25) (layer F.Cu) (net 7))
 (segment (start 165.1 118.11) (end 154.2675 118.11) (width 0.25) (layer F.Cu) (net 7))
 (segment (start 154.2675 118.11) (end 152.19 116.0325) (width 0.25) (layer F.Cu) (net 7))
 (segment (start 152.19 116.0325) (end 152.255 116.0325) (width 0.25) (layer F.Cu) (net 7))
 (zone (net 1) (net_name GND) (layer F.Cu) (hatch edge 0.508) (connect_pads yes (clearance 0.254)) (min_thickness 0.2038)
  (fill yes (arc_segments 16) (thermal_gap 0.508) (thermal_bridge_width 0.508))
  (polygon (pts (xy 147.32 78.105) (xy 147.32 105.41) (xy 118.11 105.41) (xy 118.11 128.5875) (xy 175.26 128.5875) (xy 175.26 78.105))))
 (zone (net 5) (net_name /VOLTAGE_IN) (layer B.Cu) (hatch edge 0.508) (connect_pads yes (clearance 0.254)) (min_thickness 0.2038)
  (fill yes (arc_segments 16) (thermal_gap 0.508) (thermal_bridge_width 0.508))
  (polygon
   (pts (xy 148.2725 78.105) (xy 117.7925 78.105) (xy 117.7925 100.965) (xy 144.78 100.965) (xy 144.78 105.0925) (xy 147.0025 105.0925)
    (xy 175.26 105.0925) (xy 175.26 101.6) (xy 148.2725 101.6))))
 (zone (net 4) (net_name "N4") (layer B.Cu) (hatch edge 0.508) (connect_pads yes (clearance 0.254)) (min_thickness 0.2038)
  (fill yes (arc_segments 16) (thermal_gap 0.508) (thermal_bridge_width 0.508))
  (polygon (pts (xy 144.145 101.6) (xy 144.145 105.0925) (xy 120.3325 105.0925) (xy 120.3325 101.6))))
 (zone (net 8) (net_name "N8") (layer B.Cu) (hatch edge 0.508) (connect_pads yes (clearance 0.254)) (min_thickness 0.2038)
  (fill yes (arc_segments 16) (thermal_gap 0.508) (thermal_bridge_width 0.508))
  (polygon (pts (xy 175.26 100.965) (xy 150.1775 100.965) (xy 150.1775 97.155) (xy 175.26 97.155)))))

